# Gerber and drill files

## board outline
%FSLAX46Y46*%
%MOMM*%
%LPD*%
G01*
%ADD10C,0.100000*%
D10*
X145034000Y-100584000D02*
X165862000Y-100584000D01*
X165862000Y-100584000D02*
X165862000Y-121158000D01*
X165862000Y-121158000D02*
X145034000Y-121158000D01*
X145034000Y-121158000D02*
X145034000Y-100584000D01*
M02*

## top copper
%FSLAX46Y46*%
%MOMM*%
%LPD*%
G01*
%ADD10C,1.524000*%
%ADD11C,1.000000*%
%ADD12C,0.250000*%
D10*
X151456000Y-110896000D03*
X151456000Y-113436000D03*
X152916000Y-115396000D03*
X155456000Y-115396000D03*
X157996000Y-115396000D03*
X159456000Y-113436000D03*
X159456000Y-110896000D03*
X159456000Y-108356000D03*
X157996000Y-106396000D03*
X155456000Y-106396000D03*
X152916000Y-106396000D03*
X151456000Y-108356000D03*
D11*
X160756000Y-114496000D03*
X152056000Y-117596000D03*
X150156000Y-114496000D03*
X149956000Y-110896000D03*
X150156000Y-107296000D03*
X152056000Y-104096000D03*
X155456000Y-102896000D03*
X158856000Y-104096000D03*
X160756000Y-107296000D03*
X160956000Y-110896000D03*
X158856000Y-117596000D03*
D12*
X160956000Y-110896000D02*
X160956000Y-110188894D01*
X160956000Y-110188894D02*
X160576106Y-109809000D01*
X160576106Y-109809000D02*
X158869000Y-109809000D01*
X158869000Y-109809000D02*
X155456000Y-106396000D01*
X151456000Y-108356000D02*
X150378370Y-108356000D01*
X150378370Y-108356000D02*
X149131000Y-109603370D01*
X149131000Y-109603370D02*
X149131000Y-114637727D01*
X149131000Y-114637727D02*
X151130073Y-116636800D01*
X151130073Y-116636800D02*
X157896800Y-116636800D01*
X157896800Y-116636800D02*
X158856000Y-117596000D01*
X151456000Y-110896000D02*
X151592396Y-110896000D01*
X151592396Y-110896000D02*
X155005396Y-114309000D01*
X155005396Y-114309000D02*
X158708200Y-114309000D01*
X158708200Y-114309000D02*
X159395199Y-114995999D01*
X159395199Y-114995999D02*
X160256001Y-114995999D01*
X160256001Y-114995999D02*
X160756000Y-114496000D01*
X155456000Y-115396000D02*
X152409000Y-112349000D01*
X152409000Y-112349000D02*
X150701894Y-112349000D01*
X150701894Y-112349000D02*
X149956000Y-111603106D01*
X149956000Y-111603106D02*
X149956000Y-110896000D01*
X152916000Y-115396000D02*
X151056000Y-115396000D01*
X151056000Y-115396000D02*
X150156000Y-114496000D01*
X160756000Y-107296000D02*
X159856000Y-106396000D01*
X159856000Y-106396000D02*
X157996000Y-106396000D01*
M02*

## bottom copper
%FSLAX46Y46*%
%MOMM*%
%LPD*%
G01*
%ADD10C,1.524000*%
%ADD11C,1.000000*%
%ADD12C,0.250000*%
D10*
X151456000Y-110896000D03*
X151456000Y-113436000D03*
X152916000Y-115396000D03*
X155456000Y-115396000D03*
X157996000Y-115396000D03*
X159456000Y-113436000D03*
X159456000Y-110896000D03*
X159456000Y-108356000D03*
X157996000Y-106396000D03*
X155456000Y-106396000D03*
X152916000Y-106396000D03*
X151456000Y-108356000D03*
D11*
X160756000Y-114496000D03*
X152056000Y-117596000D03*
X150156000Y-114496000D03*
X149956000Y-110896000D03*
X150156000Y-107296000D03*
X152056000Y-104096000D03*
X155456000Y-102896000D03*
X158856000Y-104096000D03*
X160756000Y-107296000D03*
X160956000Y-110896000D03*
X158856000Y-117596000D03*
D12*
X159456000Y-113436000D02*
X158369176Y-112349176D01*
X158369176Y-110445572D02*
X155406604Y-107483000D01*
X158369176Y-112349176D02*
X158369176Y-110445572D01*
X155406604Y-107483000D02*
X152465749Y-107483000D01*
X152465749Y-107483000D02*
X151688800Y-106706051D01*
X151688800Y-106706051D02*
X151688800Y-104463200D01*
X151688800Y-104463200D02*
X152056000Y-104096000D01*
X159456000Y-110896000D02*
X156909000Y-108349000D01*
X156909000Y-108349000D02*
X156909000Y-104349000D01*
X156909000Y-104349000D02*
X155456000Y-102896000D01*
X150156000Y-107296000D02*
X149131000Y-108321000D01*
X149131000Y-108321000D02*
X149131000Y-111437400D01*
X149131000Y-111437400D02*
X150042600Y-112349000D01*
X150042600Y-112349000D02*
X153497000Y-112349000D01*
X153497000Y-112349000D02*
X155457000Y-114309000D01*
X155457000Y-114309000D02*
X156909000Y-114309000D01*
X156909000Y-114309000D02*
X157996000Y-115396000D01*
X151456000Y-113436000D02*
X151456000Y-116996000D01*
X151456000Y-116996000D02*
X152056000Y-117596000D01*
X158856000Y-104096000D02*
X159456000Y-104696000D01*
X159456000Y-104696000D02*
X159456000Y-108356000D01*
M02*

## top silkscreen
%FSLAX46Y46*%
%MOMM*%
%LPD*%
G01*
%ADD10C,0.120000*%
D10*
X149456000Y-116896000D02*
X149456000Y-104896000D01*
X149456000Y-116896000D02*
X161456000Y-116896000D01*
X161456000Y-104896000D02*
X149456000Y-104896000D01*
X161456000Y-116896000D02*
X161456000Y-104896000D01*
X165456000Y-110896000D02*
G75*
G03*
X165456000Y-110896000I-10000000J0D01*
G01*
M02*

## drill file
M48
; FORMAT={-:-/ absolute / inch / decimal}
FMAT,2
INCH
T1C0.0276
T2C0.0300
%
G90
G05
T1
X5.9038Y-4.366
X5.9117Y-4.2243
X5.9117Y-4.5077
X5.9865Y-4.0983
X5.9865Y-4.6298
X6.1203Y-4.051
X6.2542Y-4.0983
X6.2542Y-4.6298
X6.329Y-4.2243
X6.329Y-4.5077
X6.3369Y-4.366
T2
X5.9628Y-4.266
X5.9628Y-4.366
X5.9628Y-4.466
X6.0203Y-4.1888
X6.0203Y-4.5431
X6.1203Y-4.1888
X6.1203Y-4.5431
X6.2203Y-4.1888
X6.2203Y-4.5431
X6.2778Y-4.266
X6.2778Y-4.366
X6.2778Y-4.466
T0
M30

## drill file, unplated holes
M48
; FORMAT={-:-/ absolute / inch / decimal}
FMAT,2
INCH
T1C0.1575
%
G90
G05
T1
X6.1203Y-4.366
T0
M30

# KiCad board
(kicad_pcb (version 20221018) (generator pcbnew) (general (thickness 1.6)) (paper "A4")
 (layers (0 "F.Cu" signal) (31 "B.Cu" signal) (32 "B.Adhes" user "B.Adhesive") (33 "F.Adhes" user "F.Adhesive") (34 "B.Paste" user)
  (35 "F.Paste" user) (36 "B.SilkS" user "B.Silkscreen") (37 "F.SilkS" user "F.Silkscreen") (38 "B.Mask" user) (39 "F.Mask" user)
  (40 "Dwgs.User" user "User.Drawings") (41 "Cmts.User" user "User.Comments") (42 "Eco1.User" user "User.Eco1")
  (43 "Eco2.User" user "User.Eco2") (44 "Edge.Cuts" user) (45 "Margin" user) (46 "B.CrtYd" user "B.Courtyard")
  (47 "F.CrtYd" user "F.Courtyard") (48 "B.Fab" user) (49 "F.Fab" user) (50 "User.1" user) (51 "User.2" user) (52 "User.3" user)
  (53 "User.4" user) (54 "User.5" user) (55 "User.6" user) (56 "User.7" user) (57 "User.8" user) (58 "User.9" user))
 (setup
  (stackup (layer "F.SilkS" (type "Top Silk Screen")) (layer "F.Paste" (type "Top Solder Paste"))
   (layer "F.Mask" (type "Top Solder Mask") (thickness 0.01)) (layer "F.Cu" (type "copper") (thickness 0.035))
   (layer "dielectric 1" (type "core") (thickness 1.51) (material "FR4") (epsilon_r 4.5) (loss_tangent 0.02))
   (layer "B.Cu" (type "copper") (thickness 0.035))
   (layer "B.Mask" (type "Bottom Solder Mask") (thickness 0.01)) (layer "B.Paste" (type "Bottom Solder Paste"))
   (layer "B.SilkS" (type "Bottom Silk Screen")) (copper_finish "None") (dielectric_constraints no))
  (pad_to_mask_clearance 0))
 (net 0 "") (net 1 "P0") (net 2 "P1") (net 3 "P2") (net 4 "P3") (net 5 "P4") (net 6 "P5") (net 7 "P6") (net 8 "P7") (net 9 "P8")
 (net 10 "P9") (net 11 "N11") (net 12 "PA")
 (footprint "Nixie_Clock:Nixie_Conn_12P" (layer "F.Cu") (at 155.456 110.896)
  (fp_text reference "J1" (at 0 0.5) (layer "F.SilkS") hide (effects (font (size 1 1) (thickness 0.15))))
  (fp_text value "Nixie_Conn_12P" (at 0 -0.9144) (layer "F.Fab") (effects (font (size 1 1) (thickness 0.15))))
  (fp_line (start -6 6) (end -6 -6) (stroke (width 0.12) (type solid)) (layer "F.SilkS"))
  (fp_line (start -6 6) (end 6 6) (stroke (width 0.12) (type solid)) (layer "F.SilkS"))
  (fp_line (start 6 -6) (end -6 -6) (stroke (width 0.12) (type solid)) (layer "F.SilkS"))
  (fp_line (start 6 6) (end 6 -6) (stroke (width 0.12) (type solid)) (layer "F.SilkS"))
  (pad "0" thru_hole circle (at -4 0) (size 1.524 1.524) (drill 0.762) (layers "*.Cu" "*.Mask") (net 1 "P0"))
  (pad "1" thru_hole circle (at -4 2.54) (size 1.524 1.524) (drill 0.762) (layers "*.Cu" "*.Mask") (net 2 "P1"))
  (pad "2" thru_hole circle (at -2.54 4.5) (size 1.524 1.524) (drill 0.762) (layers "*.Cu" "*.Mask") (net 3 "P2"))
  (pad "3" thru_hole circle (at 0 4.5) (size 1.524 1.524) (drill 0.762) (layers "*.Cu" "*.Mask") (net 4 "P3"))
  (pad "4" thru_hole circle (at 2.54 4.5) (size 1.524 1.524) (drill 0.762) (layers "*.Cu" "*.Mask") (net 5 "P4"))
  (pad "5" thru_hole circle (at 4 2.54) (size 1.524 1.524) (drill 0.762) (layers "*.Cu" "*.Mask") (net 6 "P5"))
  (pad "6" thru_hole circle (at 4 0) (size 1.524 1.524) (drill 0.762) (layers "*.Cu" "*.Mask") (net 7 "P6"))
  (pad "7" thru_hole circle (at 4 -2.54) (size 1.524 1.524) (drill 0.762) (layers "*.Cu" "*.Mask") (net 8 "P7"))
  (pad "8" thru_hole circle (at 2.54 -4.5) (size 1.524 1.524) (drill 0.762) (layers "*.Cu" "*.Mask") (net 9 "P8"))
  (pad "9" thru_hole circle (at 0 -4.5) (size 1.524 1.524) (drill 0.762) (layers "*.Cu" "*.Mask") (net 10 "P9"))
  (pad "10" thru_hole circle (at -2.54 -4.5) (size 1.524 1.524) (drill 0.762) (layers "*.Cu" "*.Mask") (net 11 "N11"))
  (pad "A" thru_hole circle (at -4 -2.54) (size 1.524 1.524) (drill 0.762) (layers "*.Cu" "*.Mask") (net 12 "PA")))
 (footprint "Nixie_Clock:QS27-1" (layer "F.Cu") (at 155.456 110.896)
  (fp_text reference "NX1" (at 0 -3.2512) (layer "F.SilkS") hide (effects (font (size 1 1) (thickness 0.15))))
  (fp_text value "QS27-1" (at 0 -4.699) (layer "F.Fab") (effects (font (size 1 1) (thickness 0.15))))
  (fp_circle (center 0 0) (end 10 0) (stroke (width 0.12) (type solid)) (fill none) (layer "F.SilkS"))
  (pad "" np_thru_hole circle (at 0 0) (size 4 4) (drill 4) (layers "*.Cu" "*.Mask"))
  (pad "0" thru_hole circle (at 5.3 3.6) (size 1 1) (drill 0.7) (layers "*.Cu" "*.Mask") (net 1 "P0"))
  (pad "1" thru_hole circle (at -3.4 6.7) (size 1 1) (drill 0.7) (layers "*.Cu" "*.Mask") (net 2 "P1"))
  (pad "2" thru_hole circle (at -5.3 3.6) (size 1 1) (drill 0.7) (layers "*.Cu" "*.Mask") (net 3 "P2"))
  (pad "3" thru_hole circle (at -5.5 0) (size 1 1) (drill 0.7) (layers "*.Cu" "*.Mask") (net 4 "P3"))
  (pad "4" thru_hole circle (at -5.3 -3.6) (size 1 1) (drill 0.7) (layers "*.Cu" "*.Mask") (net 5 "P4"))
  (pad "5" thru_hole circle (at -3.4 -6.8) (size 1 1) (drill 0.7) (layers "*.Cu" "*.Mask") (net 6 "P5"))
  (pad "6" thru_hole circle (at 0 -8) (size 1 1) (drill 0.7) (layers "*.Cu" "*.Mask") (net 7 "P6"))
  (pad "7" thru_hole circle (at 3.4 -6.8) (size 1 1) (drill 0.7) (layers "*.Cu" "*.Mask") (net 8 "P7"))
  (pad "8" thru_hole circle (at 5.3 -3.6) (size 1 1) (drill 0.7) (layers "*.Cu" "*.Mask") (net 9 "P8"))
  (pad "9" thru_hole circle (at 5.5 0) (size 1 1) (drill 0.7) (layers "*.Cu" "*.Mask") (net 10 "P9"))
  (pad "A" thru_hole circle (at 3.4 6.7) (size 1 1) (drill 0.7) (layers "*.Cu" "*.Mask") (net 12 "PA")))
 (gr_rect (start 145.034 100.584) (end 165.862 121.158) (stroke (width 0.1) (type default)) (fill none) (layer "Edge.Cuts"))
 (segment (start 150.37837 108.356) (end 149.131 109.60337) (width 0.25) (layer "F.Cu") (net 12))
 (segment (start 149.131 109.60337) (end 149.131 114.637727) (width 0.25) (layer "F.Cu") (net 12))
 (segment (start 151.130073 116.6368) (end 157.8968 116.6368) (width 0.25) (layer "F.Cu") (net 12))
 (segment (start 151.456 108.356) (end 150.37837 108.356) (width 0.25) (layer "F.Cu") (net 12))
 (segment (start 149.131 114.637727) (end 151.130073 116.6368) (width 0.25) (layer "F.Cu") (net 12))
 (segment (start 157.8968 116.6368) (end 158.856 117.596) (width 0.25) (layer "F.Cu") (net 12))
 (segment (start 155.005396 114.309) (end 158.7082 114.309) (width 0.25) (layer "F.Cu") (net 1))
 (segment (start 158.7082 114.309) (end 159.395199 114.995999) (width 0.25) (layer "F.Cu") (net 1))
 (segment (start 159.395199 114.995999) (end 160.256001 114.995999) (width 0.25) (layer "F.Cu") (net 1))
 (segment (start 160.256001 114.995999) (end 160.756 114.496) (width 0.25) (layer "F.Cu") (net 1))
 (segment (start 151.456 110.896) (end 151.592396 110.896) (width 0.25) (layer "F.Cu") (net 1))
 (segment (start 151.592396 110.896) (end 155.005396 114.309) (width 0.25) (layer "F.Cu") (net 1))
 (segment (start 151.456 113.436) (end 151.456 116.996) (width 0.25) (layer "B.Cu") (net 2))
 (segment (start 151.456 116.996) (end 152.056 117.596) (width 0.25) (layer "B.Cu") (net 2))
 (segment (start 152.916 115.396) (end 151.056 115.396) (width 0.25) (layer "F.Cu") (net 3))
 (segment (start 151.056 115.396) (end 150.156 114.496) (width 0.25) (layer "F.Cu") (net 3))
 (segment (start 155.456 115.396) (end 152.409 112.349) (width 0.25) (layer "F.Cu") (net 4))
 (segment (start 150.701894 112.349) (end 149.956 111.603106) (width 0.25) (layer "F.Cu") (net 4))
 (segment (start 149.956 111.603106) (end 149.956 110.896) (width 0.25) (layer "F.Cu") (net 4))
 (segment (start 152.409 112.349) (end 150.701894 112.349) (width 0.25) (layer "F.Cu") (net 4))
 (segment (start 150.0426 112.349) (end 153.497 112.349) (width 0.25) (layer "B.Cu") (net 5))
 (segment (start 156.909 114.309) (end 157.996 115.396) (width 0.25) (layer "B.Cu") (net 5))
 (segment (start 149.131 108.321) (end 149.131 111.4374) (width 0.25) (layer "B.Cu") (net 5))
 (segment (start 150.156 107.296) (end 149.131 108.321) (width 0.25) (layer "B.Cu") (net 5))
 (segment (start 155.457 114.309) (end 156.909 114.309) (width 0.25) (layer "B.Cu") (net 5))
 (segment (start 153.497 112.349) (end 155.457 114.309) (width 0.25) (layer "B.Cu") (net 5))
 (segment (start 149.131 111.4374) (end 150.0426 112.349) (width 0.25) (layer "B.Cu") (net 5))
 (segment (start 152.465749 107.483) (end 151.6888 106.706051) (width 0.25) (layer "B.Cu") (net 6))
 (segment (start 158.369176 110.445572) (end 155.406604 107.483) (width 0.25) (layer "B.Cu") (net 6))
 (segment (start 159.456 113.436) (end 158.369176 112.349176) (width 0.25) (layer "B.Cu") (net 6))
 (segment (start 158.369176 112.349176) (end 158.369176 110.445572) (width 0.25) (layer "B.Cu") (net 6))
 (segment (start 151.6888 106.706051) (end 151.6888 104.4632) (width 0.25) (layer "B.Cu") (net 6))
 (segment (start 155.406604 107.483) (end 152.465749 107.483) (width 0.25) (layer "B.Cu") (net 6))
 (segment (start 151.6888 104.4632) (end 152.056 104.096) (width 0.25) (layer "B.Cu") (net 6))
 (segment (start 156.909 104.349) (end 155.456 102.896) (width 0.25) (layer "B.Cu") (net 7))
 (segment (start 156.909 108.349) (end 156.909 104.349) (width 0.25) (layer "B.Cu") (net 7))
 (segment (start 159.456 110.896) (end 156.909 108.349) (width 0.25) (layer "B.Cu") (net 7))
 (segment (start 158.856 104.096) (end 159.456 104.696) (width 0.25) (layer "B.Cu") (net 8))
 (segment (start 159.456 104.696) (end 159.456 108.356) (width 0.25) (layer "B.Cu") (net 8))
 (segment (start 159.856 106.396) (end 157.996 106.396) (width 0.25) (layer "F.Cu") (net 9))
 (segment (start 160.756 107.296) (end 159.856 106.396) (width 0.25) (layer "F.Cu") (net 9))
 (segment (start 160.576106 109.809) (end 158.869 109.809) (width 0.25) (layer "F.Cu") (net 10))
 (segment (start 160.956 110.188894) (end 160.576106 109.809) (width 0.25) (layer "F.Cu") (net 10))
 (segment (start 160.956 110.896) (end 160.956 110.188894) (width 0.25) (layer "F.Cu") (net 10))
 (segment (start 158.869 109.809) (end 155.456 106.396) (width 0.25) (layer "F.Cu") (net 10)))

